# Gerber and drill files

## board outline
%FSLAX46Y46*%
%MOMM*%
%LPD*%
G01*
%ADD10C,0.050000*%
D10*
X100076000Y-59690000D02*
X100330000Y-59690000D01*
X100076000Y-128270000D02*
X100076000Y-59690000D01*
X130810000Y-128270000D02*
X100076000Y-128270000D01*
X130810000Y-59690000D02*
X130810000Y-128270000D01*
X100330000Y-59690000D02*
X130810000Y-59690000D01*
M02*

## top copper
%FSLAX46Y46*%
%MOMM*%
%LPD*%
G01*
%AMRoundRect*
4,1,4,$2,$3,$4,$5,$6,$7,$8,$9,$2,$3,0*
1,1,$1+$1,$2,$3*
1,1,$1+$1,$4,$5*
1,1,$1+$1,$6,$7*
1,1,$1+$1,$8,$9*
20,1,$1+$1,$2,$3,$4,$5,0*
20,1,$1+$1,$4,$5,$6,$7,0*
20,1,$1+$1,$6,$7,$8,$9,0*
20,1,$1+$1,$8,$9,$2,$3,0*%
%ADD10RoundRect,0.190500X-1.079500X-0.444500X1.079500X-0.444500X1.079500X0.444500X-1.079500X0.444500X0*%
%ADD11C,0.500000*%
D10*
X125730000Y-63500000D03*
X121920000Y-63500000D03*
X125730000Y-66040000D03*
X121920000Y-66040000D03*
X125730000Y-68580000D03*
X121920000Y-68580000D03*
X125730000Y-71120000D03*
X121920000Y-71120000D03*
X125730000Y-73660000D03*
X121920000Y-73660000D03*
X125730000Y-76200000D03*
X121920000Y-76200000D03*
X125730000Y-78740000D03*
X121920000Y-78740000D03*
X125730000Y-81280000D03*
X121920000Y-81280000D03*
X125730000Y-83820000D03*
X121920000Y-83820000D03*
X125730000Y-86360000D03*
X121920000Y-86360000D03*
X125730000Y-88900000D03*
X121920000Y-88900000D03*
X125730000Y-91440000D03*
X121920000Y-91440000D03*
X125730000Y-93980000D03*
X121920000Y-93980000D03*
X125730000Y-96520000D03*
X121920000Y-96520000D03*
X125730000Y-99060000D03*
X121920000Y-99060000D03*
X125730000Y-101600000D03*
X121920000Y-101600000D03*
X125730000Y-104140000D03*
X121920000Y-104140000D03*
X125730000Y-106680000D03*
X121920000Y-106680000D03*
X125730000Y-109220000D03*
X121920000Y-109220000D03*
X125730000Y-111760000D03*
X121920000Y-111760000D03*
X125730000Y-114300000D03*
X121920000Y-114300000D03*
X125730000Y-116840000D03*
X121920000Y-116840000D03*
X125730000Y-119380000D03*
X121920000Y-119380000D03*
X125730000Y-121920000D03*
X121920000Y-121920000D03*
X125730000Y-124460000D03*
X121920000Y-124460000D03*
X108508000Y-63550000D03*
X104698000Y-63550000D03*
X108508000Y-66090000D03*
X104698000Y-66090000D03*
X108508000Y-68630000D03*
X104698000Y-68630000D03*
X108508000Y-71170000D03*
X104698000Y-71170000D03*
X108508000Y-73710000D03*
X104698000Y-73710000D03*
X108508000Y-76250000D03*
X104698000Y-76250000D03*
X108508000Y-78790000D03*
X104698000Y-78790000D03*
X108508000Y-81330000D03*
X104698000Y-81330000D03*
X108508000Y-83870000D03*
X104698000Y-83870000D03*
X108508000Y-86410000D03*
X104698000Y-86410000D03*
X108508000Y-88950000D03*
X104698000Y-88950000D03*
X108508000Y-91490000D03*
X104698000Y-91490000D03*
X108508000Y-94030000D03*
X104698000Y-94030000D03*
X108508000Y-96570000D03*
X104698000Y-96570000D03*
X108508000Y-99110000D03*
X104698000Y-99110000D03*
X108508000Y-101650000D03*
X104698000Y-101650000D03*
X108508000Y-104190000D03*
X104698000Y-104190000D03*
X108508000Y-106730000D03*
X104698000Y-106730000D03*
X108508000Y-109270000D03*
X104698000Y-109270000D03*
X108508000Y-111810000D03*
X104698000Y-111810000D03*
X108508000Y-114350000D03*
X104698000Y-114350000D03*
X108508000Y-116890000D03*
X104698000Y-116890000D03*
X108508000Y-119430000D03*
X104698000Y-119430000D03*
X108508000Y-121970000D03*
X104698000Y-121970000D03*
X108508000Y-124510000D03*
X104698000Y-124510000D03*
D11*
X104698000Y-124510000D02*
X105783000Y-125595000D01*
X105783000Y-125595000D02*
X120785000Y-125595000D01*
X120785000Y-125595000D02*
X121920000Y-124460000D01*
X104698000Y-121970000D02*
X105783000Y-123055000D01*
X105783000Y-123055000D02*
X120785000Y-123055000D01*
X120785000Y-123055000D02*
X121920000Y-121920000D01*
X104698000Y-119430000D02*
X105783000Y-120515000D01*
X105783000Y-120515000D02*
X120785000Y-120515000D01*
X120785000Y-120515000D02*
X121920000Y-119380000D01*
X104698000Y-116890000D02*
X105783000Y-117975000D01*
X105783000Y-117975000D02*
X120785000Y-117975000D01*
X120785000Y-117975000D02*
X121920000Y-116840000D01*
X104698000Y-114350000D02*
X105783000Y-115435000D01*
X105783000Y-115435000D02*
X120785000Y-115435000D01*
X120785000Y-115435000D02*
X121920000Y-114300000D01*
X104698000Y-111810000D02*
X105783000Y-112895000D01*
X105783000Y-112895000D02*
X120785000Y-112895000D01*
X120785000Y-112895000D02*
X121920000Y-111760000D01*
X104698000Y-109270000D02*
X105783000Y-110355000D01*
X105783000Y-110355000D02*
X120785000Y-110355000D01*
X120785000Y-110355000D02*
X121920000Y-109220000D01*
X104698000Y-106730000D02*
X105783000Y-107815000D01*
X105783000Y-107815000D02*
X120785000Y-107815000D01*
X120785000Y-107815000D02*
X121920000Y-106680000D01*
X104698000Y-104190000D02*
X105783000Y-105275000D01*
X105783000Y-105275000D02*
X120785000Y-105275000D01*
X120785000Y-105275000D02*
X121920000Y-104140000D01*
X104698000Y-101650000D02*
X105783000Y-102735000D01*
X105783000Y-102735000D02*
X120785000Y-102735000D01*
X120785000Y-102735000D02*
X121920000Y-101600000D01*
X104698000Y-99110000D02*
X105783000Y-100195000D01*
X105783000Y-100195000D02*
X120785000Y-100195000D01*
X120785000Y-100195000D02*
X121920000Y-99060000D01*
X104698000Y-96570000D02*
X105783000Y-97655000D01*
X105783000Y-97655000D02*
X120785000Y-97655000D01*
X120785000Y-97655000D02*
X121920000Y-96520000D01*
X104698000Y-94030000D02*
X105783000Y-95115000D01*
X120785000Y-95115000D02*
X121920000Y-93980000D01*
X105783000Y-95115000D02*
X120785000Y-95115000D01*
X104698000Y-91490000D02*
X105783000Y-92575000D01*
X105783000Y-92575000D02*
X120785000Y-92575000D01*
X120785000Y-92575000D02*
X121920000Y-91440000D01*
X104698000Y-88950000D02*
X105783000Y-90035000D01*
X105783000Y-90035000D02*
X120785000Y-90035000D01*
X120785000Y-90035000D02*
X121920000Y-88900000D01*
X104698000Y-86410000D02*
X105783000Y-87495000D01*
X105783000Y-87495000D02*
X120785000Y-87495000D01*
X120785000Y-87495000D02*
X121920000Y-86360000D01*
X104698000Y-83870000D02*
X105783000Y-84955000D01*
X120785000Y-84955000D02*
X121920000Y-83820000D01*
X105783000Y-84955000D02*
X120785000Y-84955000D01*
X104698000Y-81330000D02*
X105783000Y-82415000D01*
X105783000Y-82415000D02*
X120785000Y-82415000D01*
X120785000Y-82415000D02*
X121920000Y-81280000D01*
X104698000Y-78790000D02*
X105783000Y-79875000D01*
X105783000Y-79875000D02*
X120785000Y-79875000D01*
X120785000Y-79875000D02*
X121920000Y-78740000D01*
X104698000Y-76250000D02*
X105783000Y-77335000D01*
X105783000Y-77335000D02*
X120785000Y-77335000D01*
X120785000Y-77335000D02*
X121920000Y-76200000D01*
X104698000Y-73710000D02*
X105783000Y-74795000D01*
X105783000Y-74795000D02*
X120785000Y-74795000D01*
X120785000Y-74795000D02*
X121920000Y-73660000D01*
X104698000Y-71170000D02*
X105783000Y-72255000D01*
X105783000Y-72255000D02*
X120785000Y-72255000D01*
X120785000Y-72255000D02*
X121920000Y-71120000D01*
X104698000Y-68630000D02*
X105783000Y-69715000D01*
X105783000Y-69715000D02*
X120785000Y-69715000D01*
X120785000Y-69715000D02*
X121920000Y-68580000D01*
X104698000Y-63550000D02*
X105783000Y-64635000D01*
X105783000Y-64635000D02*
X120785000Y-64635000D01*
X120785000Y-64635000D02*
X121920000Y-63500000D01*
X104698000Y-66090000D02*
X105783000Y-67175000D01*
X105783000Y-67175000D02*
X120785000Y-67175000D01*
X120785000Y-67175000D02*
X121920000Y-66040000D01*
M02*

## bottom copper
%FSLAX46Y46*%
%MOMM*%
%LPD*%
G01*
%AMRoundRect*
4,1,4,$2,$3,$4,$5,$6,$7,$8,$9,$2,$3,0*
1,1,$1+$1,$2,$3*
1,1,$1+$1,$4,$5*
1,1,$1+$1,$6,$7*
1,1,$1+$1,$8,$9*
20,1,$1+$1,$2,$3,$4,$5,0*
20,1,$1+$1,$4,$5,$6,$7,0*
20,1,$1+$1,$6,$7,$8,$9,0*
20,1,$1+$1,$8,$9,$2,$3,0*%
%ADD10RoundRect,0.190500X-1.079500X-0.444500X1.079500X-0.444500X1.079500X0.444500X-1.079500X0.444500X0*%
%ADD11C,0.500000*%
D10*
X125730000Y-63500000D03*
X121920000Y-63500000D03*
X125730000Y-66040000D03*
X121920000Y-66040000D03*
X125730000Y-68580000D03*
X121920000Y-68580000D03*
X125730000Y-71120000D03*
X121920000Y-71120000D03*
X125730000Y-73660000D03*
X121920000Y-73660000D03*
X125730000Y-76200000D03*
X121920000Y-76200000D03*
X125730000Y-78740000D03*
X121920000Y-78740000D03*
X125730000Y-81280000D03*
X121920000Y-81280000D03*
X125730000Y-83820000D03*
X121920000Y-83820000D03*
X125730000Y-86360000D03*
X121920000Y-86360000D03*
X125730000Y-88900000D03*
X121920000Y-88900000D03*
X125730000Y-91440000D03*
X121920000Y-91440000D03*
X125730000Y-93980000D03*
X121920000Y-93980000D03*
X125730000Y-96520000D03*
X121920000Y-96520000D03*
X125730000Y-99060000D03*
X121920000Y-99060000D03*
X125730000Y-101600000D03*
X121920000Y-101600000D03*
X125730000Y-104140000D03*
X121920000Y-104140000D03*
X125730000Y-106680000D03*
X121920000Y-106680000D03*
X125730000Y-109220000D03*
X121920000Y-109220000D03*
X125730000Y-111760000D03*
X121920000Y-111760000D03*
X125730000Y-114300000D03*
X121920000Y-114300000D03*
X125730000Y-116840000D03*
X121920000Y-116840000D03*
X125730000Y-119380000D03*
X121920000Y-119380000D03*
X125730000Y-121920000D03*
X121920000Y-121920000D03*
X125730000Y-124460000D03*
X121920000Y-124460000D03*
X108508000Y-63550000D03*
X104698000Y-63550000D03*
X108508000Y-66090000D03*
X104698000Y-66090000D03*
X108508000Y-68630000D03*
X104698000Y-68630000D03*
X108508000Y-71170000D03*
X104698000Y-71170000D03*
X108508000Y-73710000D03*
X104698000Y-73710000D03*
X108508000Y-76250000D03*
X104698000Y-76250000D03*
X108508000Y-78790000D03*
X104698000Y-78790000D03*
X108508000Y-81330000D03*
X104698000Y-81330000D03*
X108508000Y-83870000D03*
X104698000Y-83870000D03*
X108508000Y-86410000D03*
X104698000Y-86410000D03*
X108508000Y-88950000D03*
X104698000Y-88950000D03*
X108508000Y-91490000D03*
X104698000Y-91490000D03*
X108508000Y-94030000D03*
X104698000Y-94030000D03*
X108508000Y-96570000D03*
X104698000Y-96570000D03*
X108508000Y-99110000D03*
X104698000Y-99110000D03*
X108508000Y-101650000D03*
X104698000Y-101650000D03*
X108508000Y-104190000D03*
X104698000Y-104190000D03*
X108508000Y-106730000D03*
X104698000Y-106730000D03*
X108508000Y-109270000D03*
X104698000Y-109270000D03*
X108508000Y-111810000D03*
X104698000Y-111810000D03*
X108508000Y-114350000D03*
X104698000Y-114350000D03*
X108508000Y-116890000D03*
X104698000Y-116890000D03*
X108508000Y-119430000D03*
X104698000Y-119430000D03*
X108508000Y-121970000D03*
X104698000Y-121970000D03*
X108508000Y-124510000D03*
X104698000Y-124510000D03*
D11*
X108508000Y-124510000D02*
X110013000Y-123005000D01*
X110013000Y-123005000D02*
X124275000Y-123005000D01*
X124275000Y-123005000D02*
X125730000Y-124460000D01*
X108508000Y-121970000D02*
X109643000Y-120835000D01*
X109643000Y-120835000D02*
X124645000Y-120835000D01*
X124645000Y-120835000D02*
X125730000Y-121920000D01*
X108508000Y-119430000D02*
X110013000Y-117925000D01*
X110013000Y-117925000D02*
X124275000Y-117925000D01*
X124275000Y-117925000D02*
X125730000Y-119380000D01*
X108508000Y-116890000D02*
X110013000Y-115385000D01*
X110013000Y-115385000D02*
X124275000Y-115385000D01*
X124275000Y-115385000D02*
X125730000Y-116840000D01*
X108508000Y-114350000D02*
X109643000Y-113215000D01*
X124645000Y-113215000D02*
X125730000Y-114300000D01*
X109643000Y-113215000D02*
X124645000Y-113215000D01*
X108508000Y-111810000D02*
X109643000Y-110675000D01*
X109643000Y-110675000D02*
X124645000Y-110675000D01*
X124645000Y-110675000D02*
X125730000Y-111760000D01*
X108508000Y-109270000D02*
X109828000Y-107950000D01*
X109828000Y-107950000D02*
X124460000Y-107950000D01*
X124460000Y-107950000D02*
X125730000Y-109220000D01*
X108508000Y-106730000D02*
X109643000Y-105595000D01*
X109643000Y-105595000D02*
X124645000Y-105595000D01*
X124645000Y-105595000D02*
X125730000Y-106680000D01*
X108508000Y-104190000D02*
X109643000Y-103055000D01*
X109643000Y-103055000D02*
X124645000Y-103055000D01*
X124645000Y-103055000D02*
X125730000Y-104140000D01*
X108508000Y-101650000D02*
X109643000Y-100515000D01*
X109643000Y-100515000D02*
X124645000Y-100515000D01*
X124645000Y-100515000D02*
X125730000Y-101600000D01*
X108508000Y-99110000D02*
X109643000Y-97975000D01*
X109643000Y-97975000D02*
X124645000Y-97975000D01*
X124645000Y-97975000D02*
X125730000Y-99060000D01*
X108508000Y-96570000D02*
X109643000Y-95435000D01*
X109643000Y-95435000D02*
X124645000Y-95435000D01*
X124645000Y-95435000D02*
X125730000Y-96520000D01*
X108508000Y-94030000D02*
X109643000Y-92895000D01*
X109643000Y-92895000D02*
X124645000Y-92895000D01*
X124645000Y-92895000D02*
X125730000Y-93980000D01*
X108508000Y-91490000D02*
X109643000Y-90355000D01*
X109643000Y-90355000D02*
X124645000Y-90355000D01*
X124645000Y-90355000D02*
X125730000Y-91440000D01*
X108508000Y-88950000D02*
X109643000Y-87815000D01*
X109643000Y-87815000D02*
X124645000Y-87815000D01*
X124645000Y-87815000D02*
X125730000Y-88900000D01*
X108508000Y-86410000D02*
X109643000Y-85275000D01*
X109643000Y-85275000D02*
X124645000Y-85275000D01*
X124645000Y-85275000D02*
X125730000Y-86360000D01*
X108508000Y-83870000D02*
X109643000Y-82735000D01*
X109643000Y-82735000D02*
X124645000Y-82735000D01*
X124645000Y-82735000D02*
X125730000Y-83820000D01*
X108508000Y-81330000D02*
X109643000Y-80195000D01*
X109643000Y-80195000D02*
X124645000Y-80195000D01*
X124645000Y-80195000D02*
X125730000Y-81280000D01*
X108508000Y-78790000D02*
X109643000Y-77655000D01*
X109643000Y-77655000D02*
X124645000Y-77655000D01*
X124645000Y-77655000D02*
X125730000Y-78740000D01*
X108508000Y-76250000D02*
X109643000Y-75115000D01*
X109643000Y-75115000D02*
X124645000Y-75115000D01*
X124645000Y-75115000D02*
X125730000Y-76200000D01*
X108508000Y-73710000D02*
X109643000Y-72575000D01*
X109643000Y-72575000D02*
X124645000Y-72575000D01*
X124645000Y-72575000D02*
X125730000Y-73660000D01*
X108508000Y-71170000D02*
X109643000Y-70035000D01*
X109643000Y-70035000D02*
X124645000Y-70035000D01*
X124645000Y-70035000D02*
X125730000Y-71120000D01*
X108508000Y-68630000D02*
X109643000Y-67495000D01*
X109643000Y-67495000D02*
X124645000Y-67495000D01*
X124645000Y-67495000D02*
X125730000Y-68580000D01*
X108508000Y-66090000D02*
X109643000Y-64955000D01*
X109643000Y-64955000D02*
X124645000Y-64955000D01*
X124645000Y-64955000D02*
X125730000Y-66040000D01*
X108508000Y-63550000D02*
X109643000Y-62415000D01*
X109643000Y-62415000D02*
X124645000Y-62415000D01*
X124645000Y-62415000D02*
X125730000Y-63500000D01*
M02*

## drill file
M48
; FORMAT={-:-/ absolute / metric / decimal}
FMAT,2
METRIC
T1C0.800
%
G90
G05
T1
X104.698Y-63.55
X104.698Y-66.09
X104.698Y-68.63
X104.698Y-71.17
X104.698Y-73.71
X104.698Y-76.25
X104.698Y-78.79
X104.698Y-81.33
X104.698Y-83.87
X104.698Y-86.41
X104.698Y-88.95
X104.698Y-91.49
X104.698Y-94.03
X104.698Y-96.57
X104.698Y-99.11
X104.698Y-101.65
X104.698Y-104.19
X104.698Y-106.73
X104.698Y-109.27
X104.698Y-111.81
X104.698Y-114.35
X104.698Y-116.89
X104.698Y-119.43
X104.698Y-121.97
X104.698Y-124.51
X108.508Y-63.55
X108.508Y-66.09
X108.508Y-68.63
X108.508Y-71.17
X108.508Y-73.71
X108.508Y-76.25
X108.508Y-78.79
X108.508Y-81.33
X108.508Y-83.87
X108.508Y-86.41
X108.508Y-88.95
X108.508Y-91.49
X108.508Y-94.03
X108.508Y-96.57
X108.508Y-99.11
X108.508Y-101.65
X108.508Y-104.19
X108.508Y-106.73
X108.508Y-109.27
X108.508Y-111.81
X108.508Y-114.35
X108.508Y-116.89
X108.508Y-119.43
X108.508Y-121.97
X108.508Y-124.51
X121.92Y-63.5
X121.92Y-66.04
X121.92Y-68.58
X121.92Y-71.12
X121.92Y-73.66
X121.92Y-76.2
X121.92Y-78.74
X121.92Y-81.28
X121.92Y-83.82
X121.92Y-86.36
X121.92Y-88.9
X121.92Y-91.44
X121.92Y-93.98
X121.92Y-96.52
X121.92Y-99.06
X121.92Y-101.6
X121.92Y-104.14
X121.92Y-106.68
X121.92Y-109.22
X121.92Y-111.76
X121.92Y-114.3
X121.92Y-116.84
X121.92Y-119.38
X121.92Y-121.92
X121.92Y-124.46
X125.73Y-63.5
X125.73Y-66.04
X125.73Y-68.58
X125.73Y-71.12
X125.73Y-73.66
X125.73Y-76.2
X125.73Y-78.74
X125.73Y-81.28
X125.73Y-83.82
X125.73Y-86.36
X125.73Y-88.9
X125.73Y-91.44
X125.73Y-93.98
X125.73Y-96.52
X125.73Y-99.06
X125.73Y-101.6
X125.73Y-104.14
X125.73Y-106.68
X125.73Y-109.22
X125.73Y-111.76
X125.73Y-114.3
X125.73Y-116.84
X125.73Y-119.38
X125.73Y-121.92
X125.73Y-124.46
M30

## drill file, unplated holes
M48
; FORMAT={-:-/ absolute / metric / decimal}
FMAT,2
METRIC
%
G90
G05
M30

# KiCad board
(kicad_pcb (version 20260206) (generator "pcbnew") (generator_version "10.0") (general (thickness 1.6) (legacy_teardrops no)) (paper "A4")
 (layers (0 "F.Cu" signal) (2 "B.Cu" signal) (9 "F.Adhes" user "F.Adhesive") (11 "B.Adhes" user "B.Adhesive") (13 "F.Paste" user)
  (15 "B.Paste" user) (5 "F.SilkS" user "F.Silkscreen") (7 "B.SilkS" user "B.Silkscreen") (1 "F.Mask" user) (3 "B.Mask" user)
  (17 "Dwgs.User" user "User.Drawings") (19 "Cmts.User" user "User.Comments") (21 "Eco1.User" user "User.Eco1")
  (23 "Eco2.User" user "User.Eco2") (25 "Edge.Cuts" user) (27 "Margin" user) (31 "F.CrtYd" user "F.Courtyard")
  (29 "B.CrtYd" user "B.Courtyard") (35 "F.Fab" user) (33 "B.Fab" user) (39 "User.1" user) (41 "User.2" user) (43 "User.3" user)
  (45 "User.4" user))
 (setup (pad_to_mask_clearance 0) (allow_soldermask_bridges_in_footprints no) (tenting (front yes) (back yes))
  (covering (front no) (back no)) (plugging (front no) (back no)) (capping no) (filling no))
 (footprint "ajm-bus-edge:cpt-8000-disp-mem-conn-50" (layer "F.Cu") (at 104.19 74.726)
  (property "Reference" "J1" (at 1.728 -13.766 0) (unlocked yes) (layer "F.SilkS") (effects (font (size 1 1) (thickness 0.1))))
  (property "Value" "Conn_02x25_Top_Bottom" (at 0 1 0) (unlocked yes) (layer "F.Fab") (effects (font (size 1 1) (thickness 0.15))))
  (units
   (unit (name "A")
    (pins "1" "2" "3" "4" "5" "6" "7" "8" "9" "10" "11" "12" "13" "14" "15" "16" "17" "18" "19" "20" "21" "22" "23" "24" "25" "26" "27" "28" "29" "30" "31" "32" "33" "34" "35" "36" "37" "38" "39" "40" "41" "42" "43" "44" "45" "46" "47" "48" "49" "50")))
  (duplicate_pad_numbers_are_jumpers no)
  (pad "1" thru_hole roundrect (at 4.318 -11.176) (size 2.54 1.27) (drill 0.8) (layers "*.Cu" "*.Mask") (remove_unused_layers no)
   (roundrect_rratio 0.15) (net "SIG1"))
  (pad "2" thru_hole roundrect (at 0.508 -11.176) (size 2.54 1.27) (drill 0.8) (layers "*.Cu" "*.Mask") (remove_unused_layers no)
   (roundrect_rratio 0.15) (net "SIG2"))
  (pad "3" thru_hole roundrect (at 4.318 -8.636) (size 2.54 1.27) (drill 0.8) (layers "*.Cu" "*.Mask") (remove_unused_layers no)
   (roundrect_rratio 0.15) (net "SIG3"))
  (pad "4" thru_hole roundrect (at 0.508 -8.636) (size 2.54 1.27) (drill 0.8) (layers "*.Cu" "*.Mask") (remove_unused_layers no)
   (roundrect_rratio 0.15) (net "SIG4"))
  (pad "5" thru_hole roundrect (at 4.318 -6.096) (size 2.54 1.27) (drill 0.8) (layers "*.Cu" "*.Mask") (remove_unused_layers no)
   (roundrect_rratio 0.15) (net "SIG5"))
  (pad "6" thru_hole roundrect (at 0.508 -6.096) (size 2.54 1.27) (drill 0.8) (layers "*.Cu" "*.Mask") (remove_unused_layers no)
   (roundrect_rratio 0.15) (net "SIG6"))
  (pad "7" thru_hole roundrect (at 4.318 -3.556) (size 2.54 1.27) (drill 0.8) (layers "*.Cu" "*.Mask") (remove_unused_layers no)
   (roundrect_rratio 0.15) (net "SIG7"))
  (pad "8" thru_hole roundrect (at 0.508 -3.556) (size 2.54 1.27) (drill 0.8) (layers "*.Cu" "*.Mask") (remove_unused_layers no)
   (roundrect_rratio 0.15) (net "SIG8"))
  (pad "9" thru_hole roundrect (at 4.318 -1.016) (size 2.54 1.27) (drill 0.8) (layers "*.Cu" "*.Mask") (remove_unused_layers no)
   (roundrect_rratio 0.15) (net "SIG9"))
  (pad "10" thru_hole roundrect (at 0.508 -1.016) (size 2.54 1.27) (drill 0.8) (layers "*.Cu" "*.Mask") (remove_unused_layers no)
   (roundrect_rratio 0.15) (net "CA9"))
  (pad "11" thru_hole roundrect (at 4.318 1.524) (size 2.54 1.27) (drill 0.8) (layers "*.Cu" "*.Mask") (remove_unused_layers no)
   (roundrect_rratio 0.15) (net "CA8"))
  (pad "12" thru_hole roundrect (at 0.508 1.524) (size 2.54 1.27) (drill 0.8) (layers "*.Cu" "*.Mask") (remove_unused_layers no)
   (roundrect_rratio 0.15) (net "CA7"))
  (pad "13" thru_hole roundrect (at 4.318 4.064) (size 2.54 1.27) (drill 0.8) (layers "*.Cu" "*.Mask") (remove_unused_layers no)
   (roundrect_rratio 0.15) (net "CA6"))
  (pad "14" thru_hole roundrect (at 0.508 4.064) (size 2.54 1.27) (drill 0.8) (layers "*.Cu" "*.Mask") (remove_unused_layers no)
   (roundrect_rratio 0.15) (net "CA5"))
  (pad "15" thru_hole roundrect (at 4.318 6.604) (size 2.54 1.27) (drill 0.8) (layers "*.Cu" "*.Mask") (remove_unused_layers no)
   (roundrect_rratio 0.15) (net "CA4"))
  (pad "16" thru_hole roundrect (at 0.508 6.604) (size 2.54 1.27) (drill 0.8) (layers "*.Cu" "*.Mask") (remove_unused_layers no)
   (roundrect_rratio 0.15) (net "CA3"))
  (pad "17" thru_hole roundrect (at 4.318 9.144) (size 2.54 1.27) (drill 0.8) (layers "*.Cu" "*.Mask") (remove_unused_layers no)
   (roundrect_rratio 0.15) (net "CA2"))
  (pad "18" thru_hole roundrect (at 0.508 9.144) (size 2.54 1.27) (drill 0.8) (layers "*.Cu" "*.Mask") (remove_unused_layers no)
   (roundrect_rratio 0.15) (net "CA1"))
  (pad "19" thru_hole roundrect (at 4.318 11.684) (size 2.54 1.27) (drill 0.8) (layers "*.Cu" "*.Mask") (remove_unused_layers no)
   (roundrect_rratio 0.15) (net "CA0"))
  (pad "20" thru_hole roundrect (at 0.508 11.684) (size 2.54 1.27) (drill 0.8) (layers "*.Cu" "*.Mask") (remove_unused_layers no)
   (roundrect_rratio 0.15) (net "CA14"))
  (pad "21" thru_hole roundrect (at 4.318 14.224) (size 2.54 1.27) (drill 0.8) (layers "*.Cu" "*.Mask") (remove_unused_layers no)
   (roundrect_rratio 0.15) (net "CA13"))
  (pad "22" thru_hole roundrect (at 0.508 14.224) (size 2.54 1.27) (drill 0.8) (layers "*.Cu" "*.Mask") (remove_unused_layers no)
   (roundrect_rratio 0.15) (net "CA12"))
  (pad "23" thru_hole roundrect (at 4.318 16.764) (size 2.54 1.27) (drill 0.8) (layers "*.Cu" "*.Mask") (remove_unused_layers no)
   (roundrect_rratio 0.15) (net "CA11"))
  (pad "24" thru_hole roundrect (at 0.508 16.764) (size 2.54 1.27) (drill 0.8) (layers "*.Cu" "*.Mask") (remove_unused_layers no)
   (roundrect_rratio 0.15) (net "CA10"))
  (pad "25" thru_hole roundrect (at 4.318 19.304) (size 2.54 1.27) (drill 0.8) (layers "*.Cu" "*.Mask") (remove_unused_layers no)
   (roundrect_rratio 0.15) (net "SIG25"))
  (pad "26" thru_hole roundrect (at 0.508 19.304) (size 2.54 1.27) (drill 0.8) (layers "*.Cu" "*.Mask") (remove_unused_layers no)
   (roundrect_rratio 0.15) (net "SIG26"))
  (pad "27" thru_hole roundrect (at 4.318 21.844) (size 2.54 1.27) (drill 0.8) (layers "*.Cu" "*.Mask") (remove_unused_layers no)
   (roundrect_rratio 0.15) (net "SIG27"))
  (pad "28" thru_hole roundrect (at 0.508 21.844) (size 2.54 1.27) (drill 0.8) (layers "*.Cu" "*.Mask") (remove_unused_layers no)
   (roundrect_rratio 0.15) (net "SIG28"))
  (pad "29" thru_hole roundrect (at 4.318 24.384) (size 2.54 1.27) (drill 0.8) (layers "*.Cu" "*.Mask") (remove_unused_layers no)
   (roundrect_rratio 0.15) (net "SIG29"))
  (pad "30" thru_hole roundrect (at 0.508 24.384) (size 2.54 1.27) (drill 0.8) (layers "*.Cu" "*.Mask") (remove_unused_layers no)
   (roundrect_rratio 0.15) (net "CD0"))
  (pad "31" thru_hole roundrect (at 4.318 26.924) (size 2.54 1.27) (drill 0.8) (layers "*.Cu" "*.Mask") (remove_unused_layers no)
   (roundrect_rratio 0.15) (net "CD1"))
  (pad "32" thru_hole roundrect (at 0.508 26.924) (size 2.54 1.27) (drill 0.8) (layers "*.Cu" "*.Mask") (remove_unused_layers no)
   (roundrect_rratio 0.15) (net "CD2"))
  (pad "33" thru_hole roundrect (at 4.318 29.464) (size 2.54 1.27) (drill 0.8) (layers "*.Cu" "*.Mask") (remove_unused_layers no)
   (roundrect_rratio 0.15) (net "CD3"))
  (pad "34" thru_hole roundrect (at 0.508 29.464) (size 2.54 1.27) (drill 0.8) (layers "*.Cu" "*.Mask") (remove_unused_layers no)
   (roundrect_rratio 0.15) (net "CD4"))
  (pad "35" thru_hole roundrect (at 4.318 32.004) (size 2.54 1.27) (drill 0.8) (layers "*.Cu" "*.Mask") (remove_unused_layers no)
   (roundrect_rratio 0.15) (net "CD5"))
  (pad "36" thru_hole roundrect (at 0.508 32.004) (size 2.54 1.27) (drill 0.8) (layers "*.Cu" "*.Mask") (remove_unused_layers no)
   (roundrect_rratio 0.15) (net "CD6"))
  (pad "37" thru_hole roundrect (at 4.318 34.544) (size 2.54 1.27) (drill 0.8) (layers "*.Cu" "*.Mask") (remove_unused_layers no)
   (roundrect_rratio 0.15) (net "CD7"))
  (pad "38" thru_hole roundrect (at 0.508 34.544) (size 2.54 1.27) (drill 0.8) (layers "*.Cu" "*.Mask") (remove_unused_layers no)
   (roundrect_rratio 0.15) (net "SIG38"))
  (pad "39" thru_hole roundrect (at 4.318 37.084) (size 2.54 1.27) (drill 0.8) (layers "*.Cu" "*.Mask") (remove_unused_layers no)
   (roundrect_rratio 0.15) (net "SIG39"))
  (pad "40" thru_hole roundrect (at 0.508 37.084) (size 2.54 1.27) (drill 0.8) (layers "*.Cu" "*.Mask") (remove_unused_layers no)
   (roundrect_rratio 0.15) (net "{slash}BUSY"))
  (pad "41" thru_hole roundrect (at 4.318 39.624) (size 2.54 1.27) (drill 0.8) (layers "*.Cu" "*.Mask") (remove_unused_layers no)
   (roundrect_rratio 0.15) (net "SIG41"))
  (pad "42" thru_hole roundrect (at 0.508 39.624) (size 2.54 1.27) (drill 0.8) (layers "*.Cu" "*.Mask") (remove_unused_layers no)
   (roundrect_rratio 0.15) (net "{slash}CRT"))
  (pad "43" thru_hole roundrect (at 4.318 42.164) (size 2.54 1.27) (drill 0.8) (layers "*.Cu" "*.Mask") (remove_unused_layers no)
   (roundrect_rratio 0.15) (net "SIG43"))
  (pad "44" thru_hole roundrect (at 0.508 42.164) (size 2.54 1.27) (drill 0.8) (layers "*.Cu" "*.Mask") (remove_unused_layers no)
   (roundrect_rratio 0.15) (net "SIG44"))
  (pad "45" thru_hole roundrect (at 4.318 44.704) (size 2.54 1.27) (drill 0.8) (layers "*.Cu" "*.Mask") (remove_unused_layers no)
   (roundrect_rratio 0.15) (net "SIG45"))
  (pad "46" thru_hole roundrect (at 0.508 44.704) (size 2.54 1.27) (drill 0.8) (layers "*.Cu" "*.Mask") (remove_unused_layers no)
   (roundrect_rratio 0.15) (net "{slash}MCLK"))
  (pad "47" thru_hole roundrect (at 4.318 47.244) (size 2.54 1.27) (drill 0.8) (layers "*.Cu" "*.Mask") (remove_unused_layers no)
   (roundrect_rratio 0.15) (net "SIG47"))
  (pad "48" thru_hole roundrect (at 0.508 47.244) (size 2.54 1.27) (drill 0.8) (layers "*.Cu" "*.Mask") (remove_unused_layers no)
   (roundrect_rratio 0.15) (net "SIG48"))
  (pad "49" thru_hole roundrect (at 4.318 49.784) (size 2.54 1.27) (drill 0.8) (layers "*.Cu" "*.Mask") (remove_unused_layers no)
   (roundrect_rratio 0.15) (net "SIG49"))
  (pad "50" thru_hole roundrect (at 0.508 49.784) (size 2.54 1.27) (drill 0.8) (layers "*.Cu" "*.Mask") (remove_unused_layers no)
   (roundrect_rratio 0.15) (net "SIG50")))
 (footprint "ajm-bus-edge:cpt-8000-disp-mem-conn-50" (layer "F.Cu") (at 121.412 74.676)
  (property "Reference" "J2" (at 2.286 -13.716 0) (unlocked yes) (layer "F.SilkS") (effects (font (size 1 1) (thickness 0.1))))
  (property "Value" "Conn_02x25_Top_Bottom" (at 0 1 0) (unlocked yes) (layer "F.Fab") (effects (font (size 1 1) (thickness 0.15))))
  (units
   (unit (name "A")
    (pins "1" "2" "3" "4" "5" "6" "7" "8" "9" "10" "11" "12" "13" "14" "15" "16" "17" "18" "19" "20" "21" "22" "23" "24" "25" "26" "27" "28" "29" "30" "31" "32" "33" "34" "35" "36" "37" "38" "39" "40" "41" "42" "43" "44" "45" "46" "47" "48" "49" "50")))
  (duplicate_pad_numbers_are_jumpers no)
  (pad "1" thru_hole roundrect (at 4.318 -11.176) (size 2.54 1.27) (drill 0.8) (layers "*.Cu" "*.Mask") (remove_unused_layers no)
   (roundrect_rratio 0.15) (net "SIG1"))
  (pad "2" thru_hole roundrect (at 0.508 -11.176) (size 2.54 1.27) (drill 0.8) (layers "*.Cu" "*.Mask") (remove_unused_layers no)
   (roundrect_rratio 0.15) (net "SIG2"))
  (pad "3" thru_hole roundrect (at 4.318 -8.636) (size 2.54 1.27) (drill 0.8) (layers "*.Cu" "*.Mask") (remove_unused_layers no)
   (roundrect_rratio 0.15) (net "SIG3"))
  (pad "4" thru_hole roundrect (at 0.508 -8.636) (size 2.54 1.27) (drill 0.8) (layers "*.Cu" "*.Mask") (remove_unused_layers no)
   (roundrect_rratio 0.15) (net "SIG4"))
  (pad "5" thru_hole roundrect (at 4.318 -6.096) (size 2.54 1.27) (drill 0.8) (layers "*.Cu" "*.Mask") (remove_unused_layers no)
   (roundrect_rratio 0.15) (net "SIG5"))
  (pad "6" thru_hole roundrect (at 0.508 -6.096) (size 2.54 1.27) (drill 0.8) (layers "*.Cu" "*.Mask") (remove_unused_layers no)
   (roundrect_rratio 0.15) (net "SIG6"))
  (pad "7" thru_hole roundrect (at 4.318 -3.556) (size 2.54 1.27) (drill 0.8) (layers "*.Cu" "*.Mask") (remove_unused_layers no)
   (roundrect_rratio 0.15) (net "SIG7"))
  (pad "8" thru_hole roundrect (at 0.508 -3.556) (size 2.54 1.27) (drill 0.8) (layers "*.Cu" "*.Mask") (remove_unused_layers no)
   (roundrect_rratio 0.15) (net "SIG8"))
  (pad "9" thru_hole roundrect (at 4.318 -1.016) (size 2.54 1.27) (drill 0.8) (layers "*.Cu" "*.Mask") (remove_unused_layers no)
   (roundrect_rratio 0.15) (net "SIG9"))
  (pad "10" thru_hole roundrect (at 0.508 -1.016) (size 2.54 1.27) (drill 0.8) (layers "*.Cu" "*.Mask") (remove_unused_layers no)
   (roundrect_rratio 0.15) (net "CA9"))
  (pad "11" thru_hole roundrect (at 4.318 1.524) (size 2.54 1.27) (drill 0.8) (layers "*.Cu" "*.Mask") (remove_unused_layers no)
   (roundrect_rratio 0.15) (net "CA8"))
  (pad "12" thru_hole roundrect (at 0.508 1.524) (size 2.54 1.27) (drill 0.8) (layers "*.Cu" "*.Mask") (remove_unused_layers no)
   (roundrect_rratio 0.15) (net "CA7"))
  (pad "13" thru_hole roundrect (at 4.318 4.064) (size 2.54 1.27) (drill 0.8) (layers "*.Cu" "*.Mask") (remove_unused_layers no)
   (roundrect_rratio 0.15) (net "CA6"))
  (pad "14" thru_hole roundrect (at 0.508 4.064) (size 2.54 1.27) (drill 0.8) (layers "*.Cu" "*.Mask") (remove_unused_layers no)
   (roundrect_rratio 0.15) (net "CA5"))
  (pad "15" thru_hole roundrect (at 4.318 6.604) (size 2.54 1.27) (drill 0.8) (layers "*.Cu" "*.Mask") (remove_unused_layers no)
   (roundrect_rratio 0.15) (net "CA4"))
  (pad "16" thru_hole roundrect (at 0.508 6.604) (size 2.54 1.27) (drill 0.8) (layers "*.Cu" "*.Mask") (remove_unused_layers no)
   (roundrect_rratio 0.15) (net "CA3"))
  (pad "17" thru_hole roundrect (at 4.318 9.144) (size 2.54 1.27) (drill 0.8) (layers "*.Cu" "*.Mask") (remove_unused_layers no)
   (roundrect_rratio 0.15) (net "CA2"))
  (pad "18" thru_hole roundrect (at 0.508 9.144) (size 2.54 1.27) (drill 0.8) (layers "*.Cu" "*.Mask") (remove_unused_layers no)
   (roundrect_rratio 0.15) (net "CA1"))
  (pad "19" thru_hole roundrect (at 4.318 11.684) (size 2.54 1.27) (drill 0.8) (layers "*.Cu" "*.Mask") (remove_unused_layers no)
   (roundrect_rratio 0.15) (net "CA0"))
  (pad "20" thru_hole roundrect (at 0.508 11.684) (size 2.54 1.27) (drill 0.8) (layers "*.Cu" "*.Mask") (remove_unused_layers no)
   (roundrect_rratio 0.15) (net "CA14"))
  (pad "21" thru_hole roundrect (at 4.318 14.224) (size 2.54 1.27) (drill 0.8) (layers "*.Cu" "*.Mask") (remove_unused_layers no)
   (roundrect_rratio 0.15) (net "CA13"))
  (pad "22" thru_hole roundrect (at 0.508 14.224) (size 2.54 1.27) (drill 0.8) (layers "*.Cu" "*.Mask") (remove_unused_layers no)
   (roundrect_rratio 0.15) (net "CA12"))
  (pad "23" thru_hole roundrect (at 4.318 16.764) (size 2.54 1.27) (drill 0.8) (layers "*.Cu" "*.Mask") (remove_unused_layers no)
   (roundrect_rratio 0.15) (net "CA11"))
  (pad "24" thru_hole roundrect (at 0.508 16.764) (size 2.54 1.27) (drill 0.8) (layers "*.Cu" "*.Mask") (remove_unused_layers no)
   (roundrect_rratio 0.15) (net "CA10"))
  (pad "25" thru_hole roundrect (at 4.318 19.304) (size 2.54 1.27) (drill 0.8) (layers "*.Cu" "*.Mask") (remove_unused_layers no)
   (roundrect_rratio 0.15) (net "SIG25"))
  (pad "26" thru_hole roundrect (at 0.508 19.304) (size 2.54 1.27) (drill 0.8) (layers "*.Cu" "*.Mask") (remove_unused_layers no)
   (roundrect_rratio 0.15) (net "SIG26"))
  (pad "27" thru_hole roundrect (at 4.318 21.844) (size 2.54 1.27) (drill 0.8) (layers "*.Cu" "*.Mask") (remove_unused_layers no)
   (roundrect_rratio 0.15) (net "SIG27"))
  (pad "28" thru_hole roundrect (at 0.508 21.844) (size 2.54 1.27) (drill 0.8) (layers "*.Cu" "*.Mask") (remove_unused_layers no)
   (roundrect_rratio 0.15) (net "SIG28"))
  (pad "29" thru_hole roundrect (at 4.318 24.384) (size 2.54 1.27) (drill 0.8) (layers "*.Cu" "*.Mask") (remove_unused_layers no)
   (roundrect_rratio 0.15) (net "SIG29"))
  (pad "30" thru_hole roundrect (at 0.508 24.384) (size 2.54 1.27) (drill 0.8) (layers "*.Cu" "*.Mask") (remove_unused_layers no)
   (roundrect_rratio 0.15) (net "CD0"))
  (pad "31" thru_hole roundrect (at 4.318 26.924) (size 2.54 1.27) (drill 0.8) (layers "*.Cu" "*.Mask") (remove_unused_layers no)
   (roundrect_rratio 0.15) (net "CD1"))
  (pad "32" thru_hole roundrect (at 0.508 26.924) (size 2.54 1.27) (drill 0.8) (layers "*.Cu" "*.Mask") (remove_unused_layers no)
   (roundrect_rratio 0.15) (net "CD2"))
  (pad "33" thru_hole roundrect (at 4.318 29.464) (size 2.54 1.27) (drill 0.8) (layers "*.Cu" "*.Mask") (remove_unused_layers no)
   (roundrect_rratio 0.15) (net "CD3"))
  (pad "34" thru_hole roundrect (at 0.508 29.464) (size 2.54 1.27) (drill 0.8) (layers "*.Cu" "*.Mask") (remove_unused_layers no)
   (roundrect_rratio 0.15) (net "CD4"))
  (pad "35" thru_hole roundrect (at 4.318 32.004) (size 2.54 1.27) (drill 0.8) (layers "*.Cu" "*.Mask") (remove_unused_layers no)
   (roundrect_rratio 0.15) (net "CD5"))
  (pad "36" thru_hole roundrect (at 0.508 32.004) (size 2.54 1.27) (drill 0.8) (layers "*.Cu" "*.Mask") (remove_unused_layers no)
   (roundrect_rratio 0.15) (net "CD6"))
  (pad "37" thru_hole roundrect (at 4.318 34.544) (size 2.54 1.27) (drill 0.8) (layers "*.Cu" "*.Mask") (remove_unused_layers no)
   (roundrect_rratio 0.15) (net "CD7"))
  (pad "38" thru_hole roundrect (at 0.508 34.544) (size 2.54 1.27) (drill 0.8) (layers "*.Cu" "*.Mask") (remove_unused_layers no)
   (roundrect_rratio 0.15) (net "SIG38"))
  (pad "39" thru_hole roundrect (at 4.318 37.084) (size 2.54 1.27) (drill 0.8) (layers "*.Cu" "*.Mask") (remove_unused_layers no)
   (roundrect_rratio 0.15) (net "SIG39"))
  (pad "40" thru_hole roundrect (at 0.508 37.084) (size 2.54 1.27) (drill 0.8) (layers "*.Cu" "*.Mask") (remove_unused_layers no)
   (roundrect_rratio 0.15) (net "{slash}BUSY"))
  (pad "41" thru_hole roundrect (at 4.318 39.624) (size 2.54 1.27) (drill 0.8) (layers "*.Cu" "*.Mask") (remove_unused_layers no)
   (roundrect_rratio 0.15) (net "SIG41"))
  (pad "42" thru_hole roundrect (at 0.508 39.624) (size 2.54 1.27) (drill 0.8) (layers "*.Cu" "*.Mask") (remove_unused_layers no)
   (roundrect_rratio 0.15) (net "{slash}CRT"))
  (pad "43" thru_hole roundrect (at 4.318 42.164) (size 2.54 1.27) (drill 0.8) (layers "*.Cu" "*.Mask") (remove_unused_layers no)
   (roundrect_rratio 0.15) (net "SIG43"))
  (pad "44" thru_hole roundrect (at 0.508 42.164) (size 2.54 1.27) (drill 0.8) (layers "*.Cu" "*.Mask") (remove_unused_layers no)
   (roundrect_rratio 0.15) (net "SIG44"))
  (pad "45" thru_hole roundrect (at 4.318 44.704) (size 2.54 1.27) (drill 0.8) (layers "*.Cu" "*.Mask") (remove_unused_layers no)
   (roundrect_rratio 0.15) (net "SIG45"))
  (pad "46" thru_hole roundrect (at 0.508 44.704) (size 2.54 1.27) (drill 0.8) (layers "*.Cu" "*.Mask") (remove_unused_layers no)
   (roundrect_rratio 0.15) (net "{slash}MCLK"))
  (pad "47" thru_hole roundrect (at 4.318 47.244) (size 2.54 1.27) (drill 0.8) (layers "*.Cu" "*.Mask") (remove_unused_layers no)
   (roundrect_rratio 0.15) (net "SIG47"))
  (pad "48" thru_hole roundrect (at 0.508 47.244) (size 2.54 1.27) (drill 0.8) (layers "*.Cu" "*.Mask") (remove_unused_layers no)
   (roundrect_rratio 0.15) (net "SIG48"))
  (pad "49" thru_hole roundrect (at 4.318 49.784) (size 2.54 1.27) (drill 0.8) (layers "*.Cu" "*.Mask") (remove_unused_layers no)
   (roundrect_rratio 0.15) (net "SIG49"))
  (pad "50" thru_hole roundrect (at 0.508 49.784) (size 2.54 1.27) (drill 0.8) (layers "*.Cu" "*.Mask") (remove_unused_layers no)
   (roundrect_rratio 0.15) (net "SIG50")))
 (gr_line (start 100.076 59.69) (end 100.33 59.69) (stroke (width 0.05) (type default)) (layer "Edge.Cuts"))
 (gr_line (start 100.076 128.27) (end 100.076 59.69) (stroke (width 0.05) (type default)) (layer "Edge.Cuts"))
 (gr_line (start 100.33 59.69) (end 130.81 59.69) (stroke (width 0.05) (type default)) (layer "Edge.Cuts"))
 (gr_line (start 130.81 59.69) (end 130.81 128.27) (stroke (width 0.05) (type default)) (layer "Edge.Cuts"))
 (gr_line (start 130.81 128.27) (end 100.076 128.27) (stroke (width 0.05) (type default)) (layer "Edge.Cuts"))
 (segment (start 124.645 90.355) (end 125.73 91.44) (width 0.5) (layer "B.Cu") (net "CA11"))
 (segment (start 108.508 91.49) (end 109.643 90.355) (width 0.5) (layer "B.Cu") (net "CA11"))
 (segment (start 109.643 90.355) (end 124.645 90.355) (width 0.5) (layer "B.Cu") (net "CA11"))
 (segment (start 105.783 107.815) (end 120.785 107.815) (width 0.5) (layer "F.Cu") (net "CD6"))
 (segment (start 104.698 106.73) (end 105.783 107.815) (width 0.5) (layer "F.Cu") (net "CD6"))
 (segment (start 120.785 107.815) (end 121.92 106.68) (width 0.5) (layer "F.Cu") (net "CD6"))
 (segment (start 120.785 82.415) (end 121.92 81.28) (width 0.5) (layer "F.Cu") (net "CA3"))
 (segment (start 104.698 81.33) (end 105.783 82.415) (width 0.5) (layer "F.Cu") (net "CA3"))
 (segment (start 105.783 82.415) (end 120.785 82.415) (width 0.5) (layer "F.Cu") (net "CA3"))
 (segment (start 105.783 105.275) (end 120.785 105.275) (width 0.5) (layer "F.Cu") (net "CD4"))
 (segment (start 120.785 105.275) (end 121.92 104.14) (width 0.5) (layer "F.Cu") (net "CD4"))
 (segment (start 104.698 104.19) (end 105.783 105.275) (width 0.5) (layer "F.Cu") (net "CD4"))
 (segment (start 109.643 95.435) (end 124.645 95.435) (width 0.5) (layer "B.Cu") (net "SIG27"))
 (segment (start 108.508 96.57) (end 109.643 95.435) (width 0.5) (layer "B.Cu") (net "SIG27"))
 (segment (start 124.645 95.435) (end 125.73 96.52) (width 0.5) (layer "B.Cu") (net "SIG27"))
 (segment (start 105.783 125.595) (end 120.785 125.595) (width 0.5) (layer "F.Cu") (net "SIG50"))
 (segment (start 120.785 125.595) (end 121.92 124.46) (width 0.5) (layer "F.Cu") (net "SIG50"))
 (segment (start 104.698 124.51) (end 105.783 125.595) (width 0.5) (layer "F.Cu") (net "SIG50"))
 (segment (start 124.645 103.055) (end 125.73 104.14) (width 0.5) (layer "B.Cu") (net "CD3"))
 (segment (start 109.643 103.055) (end 124.645 103.055) (width 0.5) (layer "B.Cu") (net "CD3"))
 (segment (start 108.508 104.19) (end 109.643 103.055) (width 0.5) (layer "B.Cu") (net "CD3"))
 (segment (start 120.785 95.115) (end 121.92 93.98) (width 0.5) (layer "F.Cu") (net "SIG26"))
 (segment (start 104.698 94.03) (end 105.783 95.115) (width 0.5) (layer "F.Cu") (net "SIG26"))
 (segment (start 105.783 95.115) (end 120.785 95.115) (width 0.5) (layer "F.Cu") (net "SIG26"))
 (segment (start 120.785 72.255) (end 121.92 71.12) (width 0.5) (layer "F.Cu") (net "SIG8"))
 (segment (start 104.698 71.17) (end 105.783 72.255) (width 0.5) (layer "F.Cu") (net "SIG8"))
 (segment (start 105.783 72.255) (end 120.785 72.255) (width 0.5) (layer "F.Cu") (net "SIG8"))
 (segment (start 124.275 115.385) (end 125.73 116.84) (width 0.5) (layer "B.Cu") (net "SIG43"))
 (segment (start 110.013 115.385) (end 124.275 115.385) (width 0.5) (layer "B.Cu") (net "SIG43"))
 (segment (start 108.508 116.89) (end 110.013 115.385) (width 0.5) (layer "B.Cu") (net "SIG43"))
 (segment (start 105.783 90.035) (end 120.785 90.035) (width 0.5) (layer "F.Cu") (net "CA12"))
 (segment (start 104.698 88.95) (end 105.783 90.035) (width 0.5) (layer "F.Cu") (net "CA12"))
 (segment (start 120.785 90.035) (end 121.92 88.9) (width 0.5) (layer "F.Cu") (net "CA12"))
 (segment (start 104.698 121.97) (end 105.783 123.055) (width 0.5) (layer "F.Cu") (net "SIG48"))
 (segment (start 120.785 123.055) (end 121.92 121.92) (width 0.5) (layer "F.Cu") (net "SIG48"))
 (segment (start 105.783 123.055) (end 120.785 123.055) (width 0.5) (layer "F.Cu") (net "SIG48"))
 (segment (start 109.828 107.95) (end 124.46 107.95) (width 0.5) (layer "B.Cu") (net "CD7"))
 (segment (start 108.508 109.27) (end 109.828 107.95) (width 0.5) (layer "B.Cu") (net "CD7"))
 (segment (start 124.46 107.95) (end 125.73 109.22) (width 0.5) (layer "B.Cu") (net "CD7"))
 (segment (start 124.645 100.515) (end 125.73 101.6) (width 0.5) (layer "B.Cu") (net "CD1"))
 (segment (start 108.508 101.65) (end 109.643 100.515) (width 0.5) (layer "B.Cu") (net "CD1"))
 (segment (start 109.643 100.515) (end 124.645 100.515) (width 0.5) (layer "B.Cu") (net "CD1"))
 (segment (start 120.785 110.355) (end 121.92 109.22) (width 0.5) (layer "F.Cu") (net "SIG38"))
 (segment (start 105.783 110.355) (end 120.785 110.355) (width 0.5) (layer "F.Cu") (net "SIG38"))
 (segment (start 104.698 109.27) (end 105.783 110.355) (width 0.5) (layer "F.Cu") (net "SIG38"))
 (segment (start 120.785 79.875) (end 121.92 78.74) (width 0.5) (layer "F.Cu") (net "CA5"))
 (segment (start 105.783 79.875) (end 120.785 79.875) (width 0.5) (layer "F.Cu") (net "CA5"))
 (segment (start 104.698 78.79) (end 105.783 79.875) (width 0.5) (layer "F.Cu") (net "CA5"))
 (segment (start 124.645 70.035) (end 125.73 71.12) (width 0.5) (layer "B.Cu") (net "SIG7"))
 (segment (start 109.643 70.035) (end 124.645 70.035) (width 0.5) (layer "B.Cu") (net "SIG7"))
 (segment (start 108.508 71.17) (end 109.643 70.035) (width 0.5) (layer "B.Cu") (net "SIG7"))
 (segment (start 108.508 88.95) (end 109.643 87.815) (width 0.5) (layer "B.Cu") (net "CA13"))
 (segment (start 124.645 87.815) (end 125.73 88.9) (width 0.5) (layer "B.Cu") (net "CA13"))
 (segment (start 109.643 87.815) (end 124.645 87.815) (width 0.5) (layer "B.Cu") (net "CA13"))
 (segment (start 108.508 66.09) (end 109.643 64.955) (width 0.5) (layer "B.Cu") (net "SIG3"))
 (segment (start 109.643 64.955) (end 124.645 64.955) (width 0.5) (layer "B.Cu") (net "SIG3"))
 (segment (start 124.645 64.955) (end 125.73 66.04) (width 0.5) (layer "B.Cu") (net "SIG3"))
 (segment (start 105.783 74.795) (end 120.785 74.795) (width 0.5) (layer "F.Cu") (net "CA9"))
 (segment (start 120.785 74.795) (end 121.92 73.66) (width 0.5) (layer "F.Cu") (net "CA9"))
 (segment (start 104.698 73.71) (end 105.783 74.795) (width 0.5) (layer "F.Cu") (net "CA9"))
 (segment (start 105.783 102.735) (end 120.785 102.735) (width 0.5) (layer "F.Cu") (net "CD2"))
 (segment (start 120.785 102.735) (end 121.92 101.6) (width 0.5) (layer "F.Cu") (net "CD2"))
 (segment (start 104.698 101.65) (end 105.783 102.735) (width 0.5) (layer "F.Cu") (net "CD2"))
 (segment (start 108.508 83.87) (end 109.643 82.735) (width 0.5) (layer "B.Cu") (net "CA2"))
 (segment (start 124.645 82.735) (end 125.73 83.82) (width 0.5) (layer "B.Cu") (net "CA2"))
 (segment (start 109.643 82.735) (end 124.645 82.735) (width 0.5) (layer "B.Cu") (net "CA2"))
 (segment (start 120.785 69.715) (end 121.92 68.58) (width 0.5) (layer "F.Cu") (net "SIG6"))
 (segment (start 105.783 69.715) (end 120.785 69.715) (width 0.5) (layer "F.Cu") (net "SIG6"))
 (segment (start 104.698 68.63) (end 105.783 69.715) (width 0.5) (layer "F.Cu") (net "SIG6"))
 (segment (start 105.783 100.195) (end 120.785 100.195) (width 0.5) (layer "F.Cu") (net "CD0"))
 (segment (start 104.698 99.11) (end 105.783 100.195) (width 0.5) (layer "F.Cu") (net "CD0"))
 (segment (start 120.785 100.195) (end 121.92 99.06) (width 0.5) (layer "F.Cu") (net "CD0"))
 (segment (start 104.698 96.57) (end 105.783 97.655) (width 0.5) (layer "F.Cu") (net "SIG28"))
 (segment (start 105.783 97.655) (end 120.785 97.655) (width 0.5) (layer "F.Cu") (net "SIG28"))
 (segment (start 120.785 97.655) (end 121.92 96.52) (width 0.5) (layer "F.Cu") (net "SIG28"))
 (segment (start 108.508 106.73) (end 109.643 105.595) (width 0.5) (layer "B.Cu") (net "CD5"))
 (segment (start 109.643 105.595) (end 124.645 105.595) (width 0.5) (layer "B.Cu") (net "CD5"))
 (segment (start 124.645 105.595) (end 125.73 106.68) (width 0.5) (layer "B.Cu") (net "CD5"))
 (segment (start 105.783 112.895) (end 120.785 112.895) (width 0.5) (layer "F.Cu") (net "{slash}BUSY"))
 (segment (start 120.785 112.895) (end 121.92 111.76) (width 0.5) (layer "F.Cu") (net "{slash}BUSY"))
 (segment (start 104.698 111.81) (end 105.783 112.895) (width 0.5) (layer "F.Cu") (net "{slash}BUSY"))
 (segment (start 124.645 67.495) (end 125.73 68.58) (width 0.5) (layer "B.Cu") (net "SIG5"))
 (segment (start 108.508 68.63) (end 109.643 67.495) (width 0.5) (layer "B.Cu") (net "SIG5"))
 (segment (start 109.643 67.495) (end 124.645 67.495) (width 0.5) (layer "B.Cu") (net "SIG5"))
 (segment (start 124.645 77.655) (end 125.73 78.74) (width 0.5) (layer "B.Cu") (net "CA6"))
 (segment (start 109.643 77.655) (end 124.645 77.655) (width 0.5) (layer "B.Cu") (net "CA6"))
 (segment (start 108.508 78.79) (end 109.643 77.655) (width 0.5) (layer "B.Cu") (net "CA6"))
 (segment (start 104.698 114.35) (end 105.783 115.435) (width 0.5) (layer "F.Cu") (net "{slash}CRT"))
 (segment (start 120.785 115.435) (end 121.92 114.3) (width 0.5) (layer "F.Cu") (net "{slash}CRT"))
 (segment (start 105.783 115.435) (end 120.785 115.435) (width 0.5) (layer "F.Cu") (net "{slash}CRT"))
 (segment (start 108.508 119.43) (end 110.013 117.925) (width 0.5) (layer "B.Cu") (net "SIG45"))
 (segment (start 124.275 117.925) (end 125.73 119.38) (width 0.5) (layer "B.Cu") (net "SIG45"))
 (segment (start 110.013 117.925) (end 124.275 117.925) (width 0.5) (layer "B.Cu") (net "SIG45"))
 (segment (start 105.783 92.575) (end 120.785 92.575) (width 0.5) (layer "F.Cu") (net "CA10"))
 (segment (start 120.785 92.575) (end 121.92 91.44) (width 0.5) (layer "F.Cu") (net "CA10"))
 (segment (start 104.698 91.49) (end 105.783 92.575) (width 0.5) (layer "F.Cu") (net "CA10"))
 (segment (start 104.698 66.09) (end 105.783 67.175) (width 0.5) (layer "F.Cu") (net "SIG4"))
 (segment (start 105.783 67.175) (end 120.785 67.175) (width 0.5) (layer "F.Cu") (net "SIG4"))
 (segment (start 120.785 67.175) (end 121.92 66.04) (width 0.5) (layer "F.Cu") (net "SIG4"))
 (segment (start 109.643 72.575) (end 124.645 72.575) (width 0.5) (layer "B.Cu") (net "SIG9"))
 (segment (start 108.508 73.71) (end 109.643 72.575) (width 0.5) (layer "B.Cu") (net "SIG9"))
 (segment (start 124.645 72.575) (end 125.73 73.66) (width 0.5) (layer "B.Cu") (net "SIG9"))
 (segment (start 108.508 76.25) (end 109.643 75.115) (width 0.5) (layer "B.Cu") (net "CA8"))
 (segment (start 109.643 75.115) (end 124.645 75.115) (width 0.5) (layer "B.Cu") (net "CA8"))
 (segment (start 124.645 75.115) (end 125.73 76.2) (width 0.5) (layer "B.Cu") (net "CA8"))
 (segment (start 104.698 86.41) (end 105.783 87.495) (width 0.5) (layer "F.Cu") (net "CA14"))
 (segment (start 105.783 87.495) (end 120.785 87.495) (width 0.5) (layer "F.Cu") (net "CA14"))
 (segment (start 120.785 87.495) (end 121.92 86.36) (width 0.5) (layer "F.Cu") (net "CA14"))
 (segment (start 124.645 80.195) (end 125.73 81.28) (width 0.5) (layer "B.Cu") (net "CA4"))
 (segment (start 108.508 81.33) (end 109.643 80.195) (width 0.5) (layer "B.Cu") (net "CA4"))
 (segment (start 109.643 80.195) (end 124.645 80.195) (width 0.5) (layer "B.Cu") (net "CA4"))
 (segment (start 105.783 84.955) (end 120.785 84.955) (width 0.5) (layer "F.Cu") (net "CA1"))
 (segment (start 104.698 83.87) (end 105.783 84.955) (width 0.5) (layer "F.Cu") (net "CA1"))
 (segment (start 120.785 84.955) (end 121.92 83.82) (width 0.5) (layer "F.Cu") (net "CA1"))
 (segment (start 108.508 111.81) (end 109.643 110.675) (width 0.5) (layer "B.Cu") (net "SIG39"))
 (segment (start 124.645 110.675) (end 125.73 111.76) (width 0.5) (layer "B.Cu") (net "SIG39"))
 (segment (start 109.643 110.675) (end 124.645 110.675) (width 0.5) (layer "B.Cu") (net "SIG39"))
 (segment (start 108.508 114.35) (end 109.643 113.215) (width 0.5) (layer "B.Cu") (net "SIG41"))
 (segment (start 109.643 113.215) (end 124.645 113.215) (width 0.5) (layer "B.Cu") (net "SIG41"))
 (segment (start 124.645 113.215) (end 125.73 114.3) (width 0.5) (layer "B.Cu") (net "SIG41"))
 (segment (start 105.783 64.635) (end 120.785 64.635) (width 0.5) (layer "F.Cu") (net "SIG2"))
 (segment (start 104.698 63.55) (end 105.783 64.635) (width 0.5) (layer "F.Cu") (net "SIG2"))
 (segment (start 120.785 64.635) (end 121.92 63.5) (width 0.5) (layer "F.Cu") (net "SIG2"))
 (segment (start 124.645 92.895) (end 125.73 93.98) (width 0.5) (layer "B.Cu") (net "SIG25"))
 (segment (start 109.643 92.895) (end 124.645 92.895) (width 0.5) (layer "B.Cu") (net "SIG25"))
 (segment (start 108.508 94.03) (end 109.643 92.895) (width 0.5) (layer "B.Cu") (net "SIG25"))
 (segment (start 124.645 120.835) (end 125.73 121.92) (width 0.5) (layer "B.Cu") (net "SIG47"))
 (segment (start 109.643 120.835) (end 124.645 120.835) (width 0.5) (layer "B.Cu") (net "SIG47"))
 (segment (start 108.508 121.97) (end 109.643 120.835) (width 0.5) (layer "B.Cu") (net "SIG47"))
 (segment (start 108.508 99.11) (end 109.643 97.975) (width 0.5) (layer "B.Cu") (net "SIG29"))
 (segment (start 109.643 97.975) (end 124.645 97.975) (width 0.5) (layer "B.Cu") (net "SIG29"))
 (segment (start 124.645 97.975) (end 125.73 99.06) (width 0.5) (layer "B.Cu") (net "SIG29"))
 (segment (start 105.783 77.335) (end 120.785 77.335) (width 0.5) (layer "F.Cu") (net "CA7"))
 (segment (start 104.698 76.25) (end 105.783 77.335) (width 0.5) (layer "F.Cu") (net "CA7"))
 (segment (start 120.785 77.335) (end 121.92 76.2) (width 0.5) (layer "F.Cu") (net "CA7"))
 (segment (start 109.643 62.415) (end 124.645 62.415) (width 0.5) (layer "B.Cu") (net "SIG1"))
 (segment (start 108.508 63.55) (end 109.643 62.415) (width 0.5) (layer "B.Cu") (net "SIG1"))
 (segment (start 124.645 62.415) (end 125.73 63.5) (width 0.5) (layer "B.Cu") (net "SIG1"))
 (segment (start 105.783 117.975) (end 120.785 117.975) (width 0.5) (layer "F.Cu") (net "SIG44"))
 (segment (start 104.698 116.89) (end 105.783 117.975) (width 0.5) (layer "F.Cu") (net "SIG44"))
 (segment (start 120.785 117.975) (end 121.92 116.84) (width 0.5) (layer "F.Cu") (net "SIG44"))
 (segment (start 109.643 85.275) (end 124.645 85.275) (width 0.5) (layer "B.Cu") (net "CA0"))
 (segment (start 108.508 86.41) (end 109.643 85.275) (width 0.5) (layer "B.Cu") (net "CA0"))
 (segment (start 124.645 85.275) (end 125.73 86.36) (width 0.5) (layer "B.Cu") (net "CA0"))
 (segment (start 104.698 119.43) (end 105.783 120.515) (width 0.5) (layer "F.Cu") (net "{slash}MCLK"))
 (segment (start 120.785 120.515) (end 121.92 119.38) (width 0.5) (layer "F.Cu") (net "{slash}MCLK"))
 (segment (start 105.783 120.515) (end 120.785 120.515) (width 0.5) (layer "F.Cu") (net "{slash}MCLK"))
 (segment (start 110.013 123.005) (end 124.275 123.005) (width 0.5) (layer "B.Cu") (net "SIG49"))
 (segment (start 108.508 124.51) (end 110.013 123.005) (width 0.5) (layer "B.Cu") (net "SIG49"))
 (segment (start 124.275 123.005) (end 125.73 124.46) (width 0.5) (layer "B.Cu") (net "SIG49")))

